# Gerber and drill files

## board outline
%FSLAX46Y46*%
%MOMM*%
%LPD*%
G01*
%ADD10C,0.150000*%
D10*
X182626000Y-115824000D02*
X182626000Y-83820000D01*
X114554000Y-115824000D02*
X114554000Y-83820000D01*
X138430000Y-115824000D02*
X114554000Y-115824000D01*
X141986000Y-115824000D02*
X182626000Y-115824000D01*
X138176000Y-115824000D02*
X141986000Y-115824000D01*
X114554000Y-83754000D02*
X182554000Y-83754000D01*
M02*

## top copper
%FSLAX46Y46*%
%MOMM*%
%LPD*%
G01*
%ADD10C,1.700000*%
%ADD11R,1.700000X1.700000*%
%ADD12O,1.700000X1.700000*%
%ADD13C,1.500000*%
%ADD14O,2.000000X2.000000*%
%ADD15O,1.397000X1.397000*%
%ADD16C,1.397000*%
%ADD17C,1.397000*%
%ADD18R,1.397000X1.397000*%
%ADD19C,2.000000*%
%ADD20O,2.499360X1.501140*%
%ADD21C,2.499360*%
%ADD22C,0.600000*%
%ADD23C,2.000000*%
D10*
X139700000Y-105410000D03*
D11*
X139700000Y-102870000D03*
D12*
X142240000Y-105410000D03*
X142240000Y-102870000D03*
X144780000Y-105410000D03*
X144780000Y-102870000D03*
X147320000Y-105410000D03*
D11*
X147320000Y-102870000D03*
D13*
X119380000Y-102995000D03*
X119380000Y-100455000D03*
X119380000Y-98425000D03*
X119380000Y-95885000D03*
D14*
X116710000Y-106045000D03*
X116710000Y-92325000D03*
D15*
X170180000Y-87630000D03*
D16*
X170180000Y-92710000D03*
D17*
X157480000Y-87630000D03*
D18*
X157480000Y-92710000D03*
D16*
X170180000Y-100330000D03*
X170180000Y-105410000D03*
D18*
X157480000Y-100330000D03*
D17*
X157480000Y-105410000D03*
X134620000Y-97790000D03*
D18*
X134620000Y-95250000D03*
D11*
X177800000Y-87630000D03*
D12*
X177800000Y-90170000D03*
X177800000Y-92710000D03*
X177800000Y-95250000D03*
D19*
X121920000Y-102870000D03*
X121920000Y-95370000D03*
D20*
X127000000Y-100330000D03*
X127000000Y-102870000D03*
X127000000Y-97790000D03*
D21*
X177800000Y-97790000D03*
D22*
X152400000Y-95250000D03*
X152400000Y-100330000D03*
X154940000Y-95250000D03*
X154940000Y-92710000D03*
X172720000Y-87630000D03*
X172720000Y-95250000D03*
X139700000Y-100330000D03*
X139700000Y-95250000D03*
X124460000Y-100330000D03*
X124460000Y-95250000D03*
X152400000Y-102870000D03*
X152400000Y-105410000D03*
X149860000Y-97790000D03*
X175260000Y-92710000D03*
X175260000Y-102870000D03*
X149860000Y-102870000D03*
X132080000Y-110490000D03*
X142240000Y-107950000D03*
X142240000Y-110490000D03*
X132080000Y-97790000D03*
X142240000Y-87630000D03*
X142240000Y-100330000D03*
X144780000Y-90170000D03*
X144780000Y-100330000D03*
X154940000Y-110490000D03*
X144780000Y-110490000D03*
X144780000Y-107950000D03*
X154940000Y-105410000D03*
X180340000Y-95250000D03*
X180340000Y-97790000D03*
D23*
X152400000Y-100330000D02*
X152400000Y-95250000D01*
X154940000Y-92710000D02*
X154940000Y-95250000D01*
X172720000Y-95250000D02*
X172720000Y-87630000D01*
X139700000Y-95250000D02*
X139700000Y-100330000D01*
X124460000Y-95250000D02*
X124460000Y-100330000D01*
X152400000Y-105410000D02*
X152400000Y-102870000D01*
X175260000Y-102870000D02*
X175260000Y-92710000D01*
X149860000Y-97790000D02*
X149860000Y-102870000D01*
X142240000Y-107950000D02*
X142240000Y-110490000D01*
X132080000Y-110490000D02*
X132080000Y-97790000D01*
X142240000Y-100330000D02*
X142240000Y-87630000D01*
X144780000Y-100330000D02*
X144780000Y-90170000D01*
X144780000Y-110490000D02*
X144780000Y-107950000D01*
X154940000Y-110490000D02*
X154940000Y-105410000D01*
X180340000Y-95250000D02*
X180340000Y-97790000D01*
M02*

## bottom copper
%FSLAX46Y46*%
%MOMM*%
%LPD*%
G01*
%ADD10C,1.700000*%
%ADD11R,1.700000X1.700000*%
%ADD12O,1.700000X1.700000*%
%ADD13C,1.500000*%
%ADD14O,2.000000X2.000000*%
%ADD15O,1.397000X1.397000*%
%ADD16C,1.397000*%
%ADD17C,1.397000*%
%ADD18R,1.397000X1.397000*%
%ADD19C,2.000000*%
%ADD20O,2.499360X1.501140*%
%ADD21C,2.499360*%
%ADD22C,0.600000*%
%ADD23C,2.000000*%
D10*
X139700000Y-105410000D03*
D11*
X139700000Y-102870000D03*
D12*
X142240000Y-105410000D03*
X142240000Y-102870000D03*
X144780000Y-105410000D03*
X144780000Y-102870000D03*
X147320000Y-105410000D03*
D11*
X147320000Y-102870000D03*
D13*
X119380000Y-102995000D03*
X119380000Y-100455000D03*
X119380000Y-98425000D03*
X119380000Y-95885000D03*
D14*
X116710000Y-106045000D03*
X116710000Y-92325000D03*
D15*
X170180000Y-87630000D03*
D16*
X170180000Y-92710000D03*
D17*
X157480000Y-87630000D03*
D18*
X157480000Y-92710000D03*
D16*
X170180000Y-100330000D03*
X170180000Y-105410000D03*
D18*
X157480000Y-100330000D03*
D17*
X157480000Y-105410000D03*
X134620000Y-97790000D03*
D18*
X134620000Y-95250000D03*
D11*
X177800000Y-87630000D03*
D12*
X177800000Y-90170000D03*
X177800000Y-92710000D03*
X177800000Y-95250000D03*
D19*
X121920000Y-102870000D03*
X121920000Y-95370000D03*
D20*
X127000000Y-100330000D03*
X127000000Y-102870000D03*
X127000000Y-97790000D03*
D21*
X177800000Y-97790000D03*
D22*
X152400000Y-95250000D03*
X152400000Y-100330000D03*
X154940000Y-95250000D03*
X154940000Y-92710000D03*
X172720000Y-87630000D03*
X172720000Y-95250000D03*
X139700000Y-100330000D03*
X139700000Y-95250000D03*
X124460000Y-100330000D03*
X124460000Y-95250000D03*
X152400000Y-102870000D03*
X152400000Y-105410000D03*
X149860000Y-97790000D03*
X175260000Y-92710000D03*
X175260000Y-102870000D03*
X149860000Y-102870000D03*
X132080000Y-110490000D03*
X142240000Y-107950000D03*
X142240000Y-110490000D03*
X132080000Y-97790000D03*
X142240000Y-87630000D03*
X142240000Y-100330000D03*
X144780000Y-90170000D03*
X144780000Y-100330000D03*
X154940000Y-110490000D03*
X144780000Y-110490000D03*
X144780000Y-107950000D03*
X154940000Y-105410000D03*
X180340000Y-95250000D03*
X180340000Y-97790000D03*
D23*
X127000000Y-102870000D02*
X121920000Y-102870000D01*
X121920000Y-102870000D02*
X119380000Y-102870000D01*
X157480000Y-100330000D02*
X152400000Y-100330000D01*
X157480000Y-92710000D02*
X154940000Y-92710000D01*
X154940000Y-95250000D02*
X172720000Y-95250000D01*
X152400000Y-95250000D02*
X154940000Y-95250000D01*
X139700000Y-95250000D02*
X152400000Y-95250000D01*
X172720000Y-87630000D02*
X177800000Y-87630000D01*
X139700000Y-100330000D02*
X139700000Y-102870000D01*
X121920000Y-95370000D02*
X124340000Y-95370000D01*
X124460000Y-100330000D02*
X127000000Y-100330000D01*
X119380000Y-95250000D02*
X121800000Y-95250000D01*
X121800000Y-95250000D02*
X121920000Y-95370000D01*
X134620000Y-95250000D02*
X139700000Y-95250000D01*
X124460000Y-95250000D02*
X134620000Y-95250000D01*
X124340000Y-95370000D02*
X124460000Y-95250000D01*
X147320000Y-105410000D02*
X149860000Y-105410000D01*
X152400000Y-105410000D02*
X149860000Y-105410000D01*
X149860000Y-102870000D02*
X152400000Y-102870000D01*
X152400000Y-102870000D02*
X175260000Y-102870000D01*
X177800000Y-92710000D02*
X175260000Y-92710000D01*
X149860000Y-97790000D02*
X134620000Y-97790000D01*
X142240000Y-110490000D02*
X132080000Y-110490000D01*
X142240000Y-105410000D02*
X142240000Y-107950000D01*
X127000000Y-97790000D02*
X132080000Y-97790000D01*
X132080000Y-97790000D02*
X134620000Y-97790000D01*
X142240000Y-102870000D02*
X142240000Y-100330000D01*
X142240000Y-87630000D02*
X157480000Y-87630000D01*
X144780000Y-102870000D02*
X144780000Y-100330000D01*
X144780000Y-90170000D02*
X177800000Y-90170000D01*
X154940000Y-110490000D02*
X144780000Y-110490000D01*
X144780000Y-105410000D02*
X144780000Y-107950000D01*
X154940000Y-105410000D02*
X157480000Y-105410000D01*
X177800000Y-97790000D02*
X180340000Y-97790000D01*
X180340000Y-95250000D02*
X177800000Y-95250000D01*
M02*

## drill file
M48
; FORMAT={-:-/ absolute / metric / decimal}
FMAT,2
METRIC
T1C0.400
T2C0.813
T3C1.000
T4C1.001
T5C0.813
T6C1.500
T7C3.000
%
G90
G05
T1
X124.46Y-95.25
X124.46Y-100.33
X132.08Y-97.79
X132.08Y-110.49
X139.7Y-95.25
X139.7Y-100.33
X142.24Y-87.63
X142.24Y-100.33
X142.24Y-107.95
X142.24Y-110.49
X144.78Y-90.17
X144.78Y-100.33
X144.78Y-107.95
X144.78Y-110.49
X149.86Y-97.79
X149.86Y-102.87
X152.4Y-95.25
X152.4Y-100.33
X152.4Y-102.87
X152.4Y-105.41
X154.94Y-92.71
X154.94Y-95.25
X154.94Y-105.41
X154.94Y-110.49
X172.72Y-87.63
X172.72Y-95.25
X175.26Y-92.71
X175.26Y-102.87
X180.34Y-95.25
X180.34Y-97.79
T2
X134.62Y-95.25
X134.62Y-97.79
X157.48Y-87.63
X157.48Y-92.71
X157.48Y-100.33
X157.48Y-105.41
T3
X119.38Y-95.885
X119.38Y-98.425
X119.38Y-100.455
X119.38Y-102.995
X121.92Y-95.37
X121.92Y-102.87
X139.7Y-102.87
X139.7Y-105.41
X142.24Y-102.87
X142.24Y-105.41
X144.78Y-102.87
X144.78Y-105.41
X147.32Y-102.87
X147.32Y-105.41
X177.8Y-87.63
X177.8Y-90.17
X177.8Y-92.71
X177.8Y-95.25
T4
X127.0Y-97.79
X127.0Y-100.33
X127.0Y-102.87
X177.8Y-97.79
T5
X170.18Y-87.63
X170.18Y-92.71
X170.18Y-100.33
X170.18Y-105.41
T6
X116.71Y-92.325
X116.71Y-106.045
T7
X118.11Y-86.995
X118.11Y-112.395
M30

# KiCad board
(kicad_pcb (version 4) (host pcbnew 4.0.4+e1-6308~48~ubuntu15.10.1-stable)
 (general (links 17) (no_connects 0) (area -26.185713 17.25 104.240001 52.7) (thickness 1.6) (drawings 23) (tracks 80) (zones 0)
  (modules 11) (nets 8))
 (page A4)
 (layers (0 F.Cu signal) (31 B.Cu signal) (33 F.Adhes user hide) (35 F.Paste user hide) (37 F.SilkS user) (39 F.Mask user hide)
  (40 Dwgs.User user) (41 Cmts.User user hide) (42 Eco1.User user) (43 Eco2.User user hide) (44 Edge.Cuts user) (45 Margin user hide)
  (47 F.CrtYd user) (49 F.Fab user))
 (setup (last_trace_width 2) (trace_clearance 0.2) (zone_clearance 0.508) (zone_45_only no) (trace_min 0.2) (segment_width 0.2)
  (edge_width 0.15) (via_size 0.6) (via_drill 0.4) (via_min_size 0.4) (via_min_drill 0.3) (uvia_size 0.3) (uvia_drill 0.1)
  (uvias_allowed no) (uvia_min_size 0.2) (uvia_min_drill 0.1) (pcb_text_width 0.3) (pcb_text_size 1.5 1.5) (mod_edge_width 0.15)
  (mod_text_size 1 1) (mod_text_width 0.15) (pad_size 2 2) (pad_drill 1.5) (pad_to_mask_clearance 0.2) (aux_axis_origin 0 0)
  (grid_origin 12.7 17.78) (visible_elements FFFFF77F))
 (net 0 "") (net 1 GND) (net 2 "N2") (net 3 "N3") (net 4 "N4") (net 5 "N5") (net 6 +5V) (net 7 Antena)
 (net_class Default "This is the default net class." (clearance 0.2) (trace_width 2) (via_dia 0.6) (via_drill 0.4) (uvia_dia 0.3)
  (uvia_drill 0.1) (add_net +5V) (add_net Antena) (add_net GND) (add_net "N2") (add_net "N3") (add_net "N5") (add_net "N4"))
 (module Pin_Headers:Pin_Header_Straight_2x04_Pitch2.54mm (layer F.Cu) (at 139.7 105.41 90)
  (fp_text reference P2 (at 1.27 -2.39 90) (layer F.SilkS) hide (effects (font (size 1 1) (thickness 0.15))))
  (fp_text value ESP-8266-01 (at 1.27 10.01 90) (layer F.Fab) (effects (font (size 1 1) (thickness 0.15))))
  (pad TX thru_hole circle (at 0 0 90) (size 1.7 1.7) (drill 1) (layers *.Cu *.Mask))
  (pad 2 thru_hole rect (at 2.54 0 90) (size 1.7 1.7) (drill 1) (layers *.Cu *.Mask) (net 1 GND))
  (pad CH_P thru_hole oval (at 0 2.54 90) (size 1.7 1.7) (drill 1) (layers *.Cu *.Mask) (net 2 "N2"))
  (pad G2 thru_hole oval (at 2.54 2.54 90) (size 1.7 1.7) (drill 1) (layers *.Cu *.Mask) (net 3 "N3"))
  (pad RST thru_hole oval (at 0 5.08 90) (size 1.7 1.7) (drill 1) (layers *.Cu *.Mask) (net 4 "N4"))
  (pad G0 thru_hole oval (at 2.54 5.08 90) (size 1.7 1.7) (drill 1) (layers *.Cu *.Mask) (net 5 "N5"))
  (pad VCC thru_hole oval (at 0 7.62 90) (size 1.7 1.7) (drill 1) (layers *.Cu *.Mask) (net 2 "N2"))
  (pad RX thru_hole rect (at 2.54 7.62 90) (size 1.7 1.7) (drill 1) (layers *.Cu *.Mask)))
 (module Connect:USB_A (layer F.Cu) (at 119.38 95.885 270)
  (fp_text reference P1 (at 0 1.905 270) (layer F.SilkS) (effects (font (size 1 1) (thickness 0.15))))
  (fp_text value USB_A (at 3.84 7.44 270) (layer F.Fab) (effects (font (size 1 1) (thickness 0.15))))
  (pad 1 thru_hole circle (at 7.11 0 180) (size 1.5 1.5) (drill 1) (layers *.Cu *.Mask) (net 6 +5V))
  (pad "" thru_hole circle (at 4.57 0 180) (size 1.5 1.5) (drill 1) (layers *.Cu *.Mask))
  (pad "" thru_hole circle (at 2.54 0 180) (size 1.5 1.5) (drill 1) (layers *.Cu *.Mask))
  (pad 4 thru_hole circle (at 0 0 180) (size 1.5 1.5) (drill 1) (layers *.Cu *.Mask) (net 1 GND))
  (pad "" np_thru_hole oval (at 10.16 2.67 180) (size 2 2) (drill 1.5) (layers *.Cu *.Mask))
  (pad "" np_thru_hole oval (at -3.56 2.67 180) (size 2 2) (drill 1.5) (layers *.Cu *.Mask)))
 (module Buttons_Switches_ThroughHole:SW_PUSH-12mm (layer F.Cu) (at 163.83 90.17)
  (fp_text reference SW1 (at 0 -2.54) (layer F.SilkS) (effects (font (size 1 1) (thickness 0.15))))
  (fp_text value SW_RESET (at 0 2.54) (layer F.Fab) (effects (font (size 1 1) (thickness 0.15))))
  (pad "" np_thru_hole oval (at 6.35 -2.54) (size 1.397 1.397) (drill 0.8128) (layers *.Cu *.Mask))
  (pad "" np_thru_hole circle (at 6.35 2.54) (size 1.397 1.397) (drill 0.8128) (layers *.Cu *.Mask))
  (pad 2 thru_hole circle (at -6.35 -2.54) (size 1.397 1.397) (drill 0.8128) (layers *.Cu *.Mask) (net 3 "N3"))
  (pad 1 thru_hole rect (at -6.35 2.54) (size 1.397 1.397) (drill 0.8128) (layers *.Cu *.Mask) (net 1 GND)))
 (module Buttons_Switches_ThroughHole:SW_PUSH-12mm (layer F.Cu) (at 163.83 102.87)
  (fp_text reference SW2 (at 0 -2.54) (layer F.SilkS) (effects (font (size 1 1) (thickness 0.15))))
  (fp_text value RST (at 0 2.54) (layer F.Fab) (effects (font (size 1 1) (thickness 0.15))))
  (pad "" np_thru_hole circle (at 6.35 -2.54) (size 1.397 1.397) (drill 0.8128) (layers *.Cu *.Mask))
  (pad "" np_thru_hole circle (at 6.35 2.54) (size 1.397 1.397) (drill 0.8128) (layers *.Cu *.Mask))
  (pad 2 thru_hole rect (at -6.35 -2.54) (size 1.397 1.397) (drill 0.8128) (layers *.Cu *.Mask) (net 1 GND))
  (pad 1 thru_hole circle (at -6.35 2.54) (size 1.397 1.397) (drill 0.8128) (layers *.Cu *.Mask) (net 4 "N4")))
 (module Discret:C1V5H (layer F.Cu) (at 134.62 96.52 90)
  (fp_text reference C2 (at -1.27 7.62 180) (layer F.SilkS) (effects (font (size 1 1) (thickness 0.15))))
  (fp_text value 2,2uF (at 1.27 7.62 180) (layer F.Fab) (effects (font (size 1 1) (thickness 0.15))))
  (pad 1 thru_hole circle (at -1.27 0 90) (size 1.397 1.397) (drill 0.8128) (layers *.Cu *.Mask) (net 2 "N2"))
  (pad 2 thru_hole rect (at 1.27 0 90) (size 1.397 1.397) (drill 0.8128) (layers *.Cu *.Mask) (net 1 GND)))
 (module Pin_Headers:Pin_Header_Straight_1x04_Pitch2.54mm (layer F.Cu) (at 177.8 87.63)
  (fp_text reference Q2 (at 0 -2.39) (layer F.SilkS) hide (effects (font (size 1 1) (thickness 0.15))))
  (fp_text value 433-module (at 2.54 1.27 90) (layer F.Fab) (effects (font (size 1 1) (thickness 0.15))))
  (pad 1 thru_hole rect (at 0 0) (size 1.7 1.7) (drill 1) (layers *.Cu *.Mask) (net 1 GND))
  (pad DATA thru_hole oval (at 0 2.54) (size 1.7 1.7) (drill 1) (layers *.Cu *.Mask) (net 5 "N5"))
  (pad VCC thru_hole oval (at 0 5.08) (size 1.7 1.7) (drill 1) (layers *.Cu *.Mask) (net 2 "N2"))
  (pad 4 thru_hole oval (at 0 7.62) (size 1.7 1.7) (drill 1) (layers *.Cu *.Mask) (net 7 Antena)))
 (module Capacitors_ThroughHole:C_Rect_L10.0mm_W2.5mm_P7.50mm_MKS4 (layer F.Cu) (at 121.92 102.87 90)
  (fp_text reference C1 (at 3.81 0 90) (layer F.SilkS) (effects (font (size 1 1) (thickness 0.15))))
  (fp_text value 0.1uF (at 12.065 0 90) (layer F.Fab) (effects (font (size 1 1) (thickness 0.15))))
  (pad 1 thru_hole circle (at 0 0 90) (size 2 2) (drill 1) (layers *.Cu *.Mask) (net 6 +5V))
  (pad 2 thru_hole circle (at 7.5 0 90) (size 2 2) (drill 1) (layers *.Cu *.Mask) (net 1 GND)))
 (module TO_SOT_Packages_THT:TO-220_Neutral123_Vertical (layer F.Cu) (at 127 100.33 90)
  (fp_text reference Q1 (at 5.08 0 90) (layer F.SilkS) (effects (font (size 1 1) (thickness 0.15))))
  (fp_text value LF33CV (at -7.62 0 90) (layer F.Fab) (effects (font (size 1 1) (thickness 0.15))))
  (pad 2 thru_hole oval (at 0 0 180) (size 2.49936 1.50114) (drill 1.00076) (layers *.Cu *.Mask) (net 1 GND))
  (pad 1 thru_hole oval (at -2.54 0 180) (size 2.49936 1.50114) (drill 1.00076) (layers *.Cu *.Mask) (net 6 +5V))
  (pad 3 thru_hole oval (at 2.54 0 180) (size 2.49936 1.50114) (drill 1.00076) (layers *.Cu *.Mask) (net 2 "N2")))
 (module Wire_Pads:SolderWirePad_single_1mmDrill (layer F.Cu) (at 177.8 97.79)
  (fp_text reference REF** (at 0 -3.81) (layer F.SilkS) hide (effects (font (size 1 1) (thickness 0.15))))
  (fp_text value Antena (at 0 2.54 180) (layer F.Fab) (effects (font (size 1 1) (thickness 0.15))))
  (pad 1 thru_hole circle (at 0 0) (size 2.49936 2.49936) (drill 1.00076) (layers *.Cu *.Mask) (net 7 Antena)))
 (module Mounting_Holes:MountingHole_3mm (layer F.Cu) (at 118.11 112.395)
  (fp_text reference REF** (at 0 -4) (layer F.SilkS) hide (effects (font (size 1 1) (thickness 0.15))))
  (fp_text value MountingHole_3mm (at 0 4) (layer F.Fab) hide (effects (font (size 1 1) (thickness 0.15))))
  (pad 1 np_thru_hole circle (at 0 0) (size 3 3) (drill 3) (layers *.Cu *.Mask)))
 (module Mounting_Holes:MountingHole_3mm (layer F.Cu) (at 118.11 86.995)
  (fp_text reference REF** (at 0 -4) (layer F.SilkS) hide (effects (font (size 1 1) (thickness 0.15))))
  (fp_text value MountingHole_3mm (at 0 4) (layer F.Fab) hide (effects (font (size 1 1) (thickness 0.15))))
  (pad 1 np_thru_hole circle (at 0 0) (size 3 3) (drill 3) (layers *.Cu *.Mask)))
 (gr_line (start 182.626 115.824) (end 182.626 83.82) (angle 90) (layer Edge.Cuts) (width 0.15))
 (gr_line (start 114.554 115.824) (end 114.554 83.82) (angle 90) (layer Edge.Cuts) (width 0.15))
 (gr_line (start 138.43 115.824) (end 114.554 115.824) (angle 90) (layer Edge.Cuts) (width 0.15))
 (gr_line (start 141.986 115.824) (end 182.626 115.824) (angle 90) (layer Edge.Cuts) (width 0.15))
 (gr_line (start 138.176 115.824) (end 141.986 115.824) (angle 90) (layer Edge.Cuts) (width 0.15))
 (gr_line (start 114.554 83.754) (end 182.554 83.754) (angle 90) (layer Edge.Cuts) (width 0.15))
 (segment (start 127 102.87) (end 121.92 102.87) (width 2) (layer B.Cu) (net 6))
 (segment (start 121.92 102.87) (end 119.38 102.87) (width 2) (layer B.Cu) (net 6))
 (segment (start 157.48 100.33) (end 152.4 100.33) (width 2) (layer B.Cu) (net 1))
 (via (at 152.4 95.25) (size 0.6) (drill 0.4) (layers F.Cu B.Cu) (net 1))
 (segment (start 152.4 100.33) (end 152.4 95.25) (width 2) (layer F.Cu) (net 1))
 (via (at 152.4 100.33) (size 0.6) (drill 0.4) (layers F.Cu B.Cu) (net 1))
 (via (at 154.94 95.25) (size 0.6) (drill 0.4) (layers F.Cu B.Cu) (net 1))
 (segment (start 154.94 92.71) (end 154.94 95.25) (width 2) (layer F.Cu) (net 1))
 (via (at 154.94 92.71) (size 0.6) (drill 0.4) (layers F.Cu B.Cu) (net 1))
 (segment (start 157.48 92.71) (end 154.94 92.71) (width 2) (layer B.Cu) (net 1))
 (segment (start 154.94 95.25) (end 172.72 95.25) (width 2) (layer B.Cu) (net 1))
 (segment (start 152.4 95.25) (end 154.94 95.25) (width 2) (layer B.Cu) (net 1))
 (segment (start 139.7 95.25) (end 152.4 95.25) (width 2) (layer B.Cu) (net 1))
 (segment (start 172.72 87.63) (end 177.8 87.63) (width 2) (layer B.Cu) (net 1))
 (via (at 172.72 87.63) (size 0.6) (drill 0.4) (layers F.Cu B.Cu) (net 1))
 (segment (start 172.72 95.25) (end 172.72 87.63) (width 2) (layer F.Cu) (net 1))
 (via (at 172.72 95.25) (size 0.6) (drill 0.4) (layers F.Cu B.Cu) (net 1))
 (segment (start 139.7 100.33) (end 139.7 102.87) (width 2) (layer B.Cu) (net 1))
 (via (at 139.7 100.33) (size 0.6) (drill 0.4) (layers F.Cu B.Cu) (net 1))
 (segment (start 139.7 95.25) (end 139.7 100.33) (width 2) (layer F.Cu) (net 1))
 (via (at 139.7 95.25) (size 0.6) (drill 0.4) (layers F.Cu B.Cu) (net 1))
 (segment (start 121.92 95.37) (end 124.34 95.37) (width 2) (layer B.Cu) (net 1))
 (segment (start 124.46 100.33) (end 127 100.33) (width 2) (layer B.Cu) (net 1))
 (via (at 124.46 100.33) (size 0.6) (drill 0.4) (layers F.Cu B.Cu) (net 1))
 (segment (start 124.46 95.25) (end 124.46 100.33) (width 2) (layer F.Cu) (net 1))
 (segment (start 119.38 95.25) (end 121.8 95.25) (width 2) (layer B.Cu) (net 1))
 (segment (start 121.8 95.25) (end 121.92 95.37) (width 2) (layer B.Cu) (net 1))
 (segment (start 134.62 95.25) (end 139.7 95.25) (width 2) (layer B.Cu) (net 1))
 (segment (start 124.46 95.25) (end 134.62 95.25) (width 2) (layer B.Cu) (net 1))
 (via (at 124.46 95.25) (size 0.6) (drill 0.4) (layers F.Cu B.Cu) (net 1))
 (segment (start 124.34 95.37) (end 124.46 95.25) (width 2) (layer B.Cu) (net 1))
 (via (at 152.4 102.87) (size 0.6) (drill 0.4) (layers F.Cu B.Cu) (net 2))
 (segment (start 147.32 105.41) (end 149.86 105.41) (width 2) (layer B.Cu) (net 2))
 (segment (start 152.4 105.41) (end 149.86 105.41) (width 2) (layer B.Cu) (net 2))
 (via (at 152.4 105.41) (size 0.6) (drill 0.4) (layers F.Cu B.Cu) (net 2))
 (segment (start 152.4 105.41) (end 152.4 102.87) (width 2) (layer F.Cu) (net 2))
 (via (at 149.86 97.79) (size 0.6) (drill 0.4) (layers F.Cu B.Cu) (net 2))
 (via (at 175.26 92.71) (size 0.6) (drill 0.4) (layers F.Cu B.Cu) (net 2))
 (segment (start 175.26 102.87) (end 175.26 92.71) (width 2) (layer F.Cu) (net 2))
 (via (at 175.26 102.87) (size 0.6) (drill 0.4) (layers F.Cu B.Cu) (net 2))
 (segment (start 149.86 102.87) (end 152.4 102.87) (width 2) (layer B.Cu) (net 2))
 (segment (start 152.4 102.87) (end 175.26 102.87) (width 2) (layer B.Cu) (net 2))
 (segment (start 177.8 92.71) (end 175.26 92.71) (width 2) (layer B.Cu) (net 2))
 (segment (start 149.86 97.79) (end 134.62 97.79) (width 2) (layer B.Cu) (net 2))
 (via (at 149.86 102.87) (size 0.6) (drill 0.4) (layers F.Cu B.Cu) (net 2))
 (segment (start 149.86 97.79) (end 149.86 102.87) (width 2) (layer F.Cu) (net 2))
 (via (at 132.08 110.49) (size 0.6) (drill 0.4) (layers F.Cu B.Cu) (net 2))
 (via (at 142.24 107.95) (size 0.6) (drill 0.4) (layers F.Cu B.Cu) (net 2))
 (segment (start 142.24 107.95) (end 142.24 110.49) (width 2) (layer F.Cu) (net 2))
 (via (at 142.24 110.49) (size 0.6) (drill 0.4) (layers F.Cu B.Cu) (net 2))
 (segment (start 142.24 110.49) (end 132.08 110.49) (width 2) (layer B.Cu) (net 2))
 (segment (start 142.24 105.41) (end 142.24 107.95) (width 2) (layer B.Cu) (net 2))
 (via (at 132.08 97.79) (size 0.6) (drill 0.4) (layers F.Cu B.Cu) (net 2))
 (segment (start 132.08 110.49) (end 132.08 97.79) (width 2) (layer F.Cu) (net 2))
 (segment (start 127 97.79) (end 132.08 97.79) (width 2) (layer B.Cu) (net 2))
 (segment (start 132.08 97.79) (end 134.62 97.79) (width 2) (layer B.Cu) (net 2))
 (segment (start 142.24 102.87) (end 142.24 100.33) (width 2) (layer B.Cu) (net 3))
 (segment (start 142.24 87.63) (end 157.48 87.63) (width 2) (layer B.Cu) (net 3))
 (via (at 142.24 87.63) (size 0.6) (drill 0.4) (layers F.Cu B.Cu) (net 3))
 (segment (start 142.24 100.33) (end 142.24 87.63) (width 2) (layer F.Cu) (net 3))
 (via (at 142.24 100.33) (size 0.6) (drill 0.4) (layers F.Cu B.Cu) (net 3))
 (segment (start 144.78 102.87) (end 144.78 100.33) (width 2) (layer B.Cu) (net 5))
 (segment (start 144.78 90.17) (end 177.8 90.17) (width 2) (layer B.Cu) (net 5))
 (via (at 144.78 90.17) (size 0.6) (drill 0.4) (layers F.Cu B.Cu) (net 5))
 (segment (start 144.78 100.33) (end 144.78 90.17) (width 2) (layer F.Cu) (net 5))
 (via (at 144.78 100.33) (size 0.6) (drill 0.4) (layers F.Cu B.Cu) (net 5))
 (via (at 154.94 110.49) (size 0.6) (drill 0.4) (layers F.Cu B.Cu) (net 4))
 (segment (start 154.94 110.49) (end 144.78 110.49) (width 2) (layer B.Cu) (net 4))
 (via (at 144.78 110.49) (size 0.6) (drill 0.4) (layers F.Cu B.Cu) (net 4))
 (segment (start 144.78 110.49) (end 144.78 107.95) (width 2) (layer F.Cu) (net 4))
 (via (at 144.78 107.95) (size 0.6) (drill 0.4) (layers F.Cu B.Cu) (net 4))
 (segment (start 144.78 105.41) (end 144.78 107.95) (width 2) (layer B.Cu) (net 4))
 (segment (start 154.94 105.41) (end 157.48 105.41) (width 2) (layer B.Cu) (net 4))
 (via (at 154.94 105.41) (size 0.6) (drill 0.4) (layers F.Cu B.Cu) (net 4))
 (segment (start 154.94 110.49) (end 154.94 105.41) (width 2) (layer F.Cu) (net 4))
 (via (at 180.34 95.25) (size 0.6) (drill 0.4) (layers F.Cu B.Cu) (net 7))
 (segment (start 177.8 97.79) (end 180.34 97.79) (width 2) (layer B.Cu) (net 7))
 (segment (start 180.34 95.25) (end 177.8 95.25) (width 2) (layer B.Cu) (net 7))
 (via (at 180.34 97.79) (size 0.6) (drill 0.4) (layers F.Cu B.Cu) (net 7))
 (segment (start 180.34 95.25) (end 180.34 97.79) (width 2) (layer F.Cu) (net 7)))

